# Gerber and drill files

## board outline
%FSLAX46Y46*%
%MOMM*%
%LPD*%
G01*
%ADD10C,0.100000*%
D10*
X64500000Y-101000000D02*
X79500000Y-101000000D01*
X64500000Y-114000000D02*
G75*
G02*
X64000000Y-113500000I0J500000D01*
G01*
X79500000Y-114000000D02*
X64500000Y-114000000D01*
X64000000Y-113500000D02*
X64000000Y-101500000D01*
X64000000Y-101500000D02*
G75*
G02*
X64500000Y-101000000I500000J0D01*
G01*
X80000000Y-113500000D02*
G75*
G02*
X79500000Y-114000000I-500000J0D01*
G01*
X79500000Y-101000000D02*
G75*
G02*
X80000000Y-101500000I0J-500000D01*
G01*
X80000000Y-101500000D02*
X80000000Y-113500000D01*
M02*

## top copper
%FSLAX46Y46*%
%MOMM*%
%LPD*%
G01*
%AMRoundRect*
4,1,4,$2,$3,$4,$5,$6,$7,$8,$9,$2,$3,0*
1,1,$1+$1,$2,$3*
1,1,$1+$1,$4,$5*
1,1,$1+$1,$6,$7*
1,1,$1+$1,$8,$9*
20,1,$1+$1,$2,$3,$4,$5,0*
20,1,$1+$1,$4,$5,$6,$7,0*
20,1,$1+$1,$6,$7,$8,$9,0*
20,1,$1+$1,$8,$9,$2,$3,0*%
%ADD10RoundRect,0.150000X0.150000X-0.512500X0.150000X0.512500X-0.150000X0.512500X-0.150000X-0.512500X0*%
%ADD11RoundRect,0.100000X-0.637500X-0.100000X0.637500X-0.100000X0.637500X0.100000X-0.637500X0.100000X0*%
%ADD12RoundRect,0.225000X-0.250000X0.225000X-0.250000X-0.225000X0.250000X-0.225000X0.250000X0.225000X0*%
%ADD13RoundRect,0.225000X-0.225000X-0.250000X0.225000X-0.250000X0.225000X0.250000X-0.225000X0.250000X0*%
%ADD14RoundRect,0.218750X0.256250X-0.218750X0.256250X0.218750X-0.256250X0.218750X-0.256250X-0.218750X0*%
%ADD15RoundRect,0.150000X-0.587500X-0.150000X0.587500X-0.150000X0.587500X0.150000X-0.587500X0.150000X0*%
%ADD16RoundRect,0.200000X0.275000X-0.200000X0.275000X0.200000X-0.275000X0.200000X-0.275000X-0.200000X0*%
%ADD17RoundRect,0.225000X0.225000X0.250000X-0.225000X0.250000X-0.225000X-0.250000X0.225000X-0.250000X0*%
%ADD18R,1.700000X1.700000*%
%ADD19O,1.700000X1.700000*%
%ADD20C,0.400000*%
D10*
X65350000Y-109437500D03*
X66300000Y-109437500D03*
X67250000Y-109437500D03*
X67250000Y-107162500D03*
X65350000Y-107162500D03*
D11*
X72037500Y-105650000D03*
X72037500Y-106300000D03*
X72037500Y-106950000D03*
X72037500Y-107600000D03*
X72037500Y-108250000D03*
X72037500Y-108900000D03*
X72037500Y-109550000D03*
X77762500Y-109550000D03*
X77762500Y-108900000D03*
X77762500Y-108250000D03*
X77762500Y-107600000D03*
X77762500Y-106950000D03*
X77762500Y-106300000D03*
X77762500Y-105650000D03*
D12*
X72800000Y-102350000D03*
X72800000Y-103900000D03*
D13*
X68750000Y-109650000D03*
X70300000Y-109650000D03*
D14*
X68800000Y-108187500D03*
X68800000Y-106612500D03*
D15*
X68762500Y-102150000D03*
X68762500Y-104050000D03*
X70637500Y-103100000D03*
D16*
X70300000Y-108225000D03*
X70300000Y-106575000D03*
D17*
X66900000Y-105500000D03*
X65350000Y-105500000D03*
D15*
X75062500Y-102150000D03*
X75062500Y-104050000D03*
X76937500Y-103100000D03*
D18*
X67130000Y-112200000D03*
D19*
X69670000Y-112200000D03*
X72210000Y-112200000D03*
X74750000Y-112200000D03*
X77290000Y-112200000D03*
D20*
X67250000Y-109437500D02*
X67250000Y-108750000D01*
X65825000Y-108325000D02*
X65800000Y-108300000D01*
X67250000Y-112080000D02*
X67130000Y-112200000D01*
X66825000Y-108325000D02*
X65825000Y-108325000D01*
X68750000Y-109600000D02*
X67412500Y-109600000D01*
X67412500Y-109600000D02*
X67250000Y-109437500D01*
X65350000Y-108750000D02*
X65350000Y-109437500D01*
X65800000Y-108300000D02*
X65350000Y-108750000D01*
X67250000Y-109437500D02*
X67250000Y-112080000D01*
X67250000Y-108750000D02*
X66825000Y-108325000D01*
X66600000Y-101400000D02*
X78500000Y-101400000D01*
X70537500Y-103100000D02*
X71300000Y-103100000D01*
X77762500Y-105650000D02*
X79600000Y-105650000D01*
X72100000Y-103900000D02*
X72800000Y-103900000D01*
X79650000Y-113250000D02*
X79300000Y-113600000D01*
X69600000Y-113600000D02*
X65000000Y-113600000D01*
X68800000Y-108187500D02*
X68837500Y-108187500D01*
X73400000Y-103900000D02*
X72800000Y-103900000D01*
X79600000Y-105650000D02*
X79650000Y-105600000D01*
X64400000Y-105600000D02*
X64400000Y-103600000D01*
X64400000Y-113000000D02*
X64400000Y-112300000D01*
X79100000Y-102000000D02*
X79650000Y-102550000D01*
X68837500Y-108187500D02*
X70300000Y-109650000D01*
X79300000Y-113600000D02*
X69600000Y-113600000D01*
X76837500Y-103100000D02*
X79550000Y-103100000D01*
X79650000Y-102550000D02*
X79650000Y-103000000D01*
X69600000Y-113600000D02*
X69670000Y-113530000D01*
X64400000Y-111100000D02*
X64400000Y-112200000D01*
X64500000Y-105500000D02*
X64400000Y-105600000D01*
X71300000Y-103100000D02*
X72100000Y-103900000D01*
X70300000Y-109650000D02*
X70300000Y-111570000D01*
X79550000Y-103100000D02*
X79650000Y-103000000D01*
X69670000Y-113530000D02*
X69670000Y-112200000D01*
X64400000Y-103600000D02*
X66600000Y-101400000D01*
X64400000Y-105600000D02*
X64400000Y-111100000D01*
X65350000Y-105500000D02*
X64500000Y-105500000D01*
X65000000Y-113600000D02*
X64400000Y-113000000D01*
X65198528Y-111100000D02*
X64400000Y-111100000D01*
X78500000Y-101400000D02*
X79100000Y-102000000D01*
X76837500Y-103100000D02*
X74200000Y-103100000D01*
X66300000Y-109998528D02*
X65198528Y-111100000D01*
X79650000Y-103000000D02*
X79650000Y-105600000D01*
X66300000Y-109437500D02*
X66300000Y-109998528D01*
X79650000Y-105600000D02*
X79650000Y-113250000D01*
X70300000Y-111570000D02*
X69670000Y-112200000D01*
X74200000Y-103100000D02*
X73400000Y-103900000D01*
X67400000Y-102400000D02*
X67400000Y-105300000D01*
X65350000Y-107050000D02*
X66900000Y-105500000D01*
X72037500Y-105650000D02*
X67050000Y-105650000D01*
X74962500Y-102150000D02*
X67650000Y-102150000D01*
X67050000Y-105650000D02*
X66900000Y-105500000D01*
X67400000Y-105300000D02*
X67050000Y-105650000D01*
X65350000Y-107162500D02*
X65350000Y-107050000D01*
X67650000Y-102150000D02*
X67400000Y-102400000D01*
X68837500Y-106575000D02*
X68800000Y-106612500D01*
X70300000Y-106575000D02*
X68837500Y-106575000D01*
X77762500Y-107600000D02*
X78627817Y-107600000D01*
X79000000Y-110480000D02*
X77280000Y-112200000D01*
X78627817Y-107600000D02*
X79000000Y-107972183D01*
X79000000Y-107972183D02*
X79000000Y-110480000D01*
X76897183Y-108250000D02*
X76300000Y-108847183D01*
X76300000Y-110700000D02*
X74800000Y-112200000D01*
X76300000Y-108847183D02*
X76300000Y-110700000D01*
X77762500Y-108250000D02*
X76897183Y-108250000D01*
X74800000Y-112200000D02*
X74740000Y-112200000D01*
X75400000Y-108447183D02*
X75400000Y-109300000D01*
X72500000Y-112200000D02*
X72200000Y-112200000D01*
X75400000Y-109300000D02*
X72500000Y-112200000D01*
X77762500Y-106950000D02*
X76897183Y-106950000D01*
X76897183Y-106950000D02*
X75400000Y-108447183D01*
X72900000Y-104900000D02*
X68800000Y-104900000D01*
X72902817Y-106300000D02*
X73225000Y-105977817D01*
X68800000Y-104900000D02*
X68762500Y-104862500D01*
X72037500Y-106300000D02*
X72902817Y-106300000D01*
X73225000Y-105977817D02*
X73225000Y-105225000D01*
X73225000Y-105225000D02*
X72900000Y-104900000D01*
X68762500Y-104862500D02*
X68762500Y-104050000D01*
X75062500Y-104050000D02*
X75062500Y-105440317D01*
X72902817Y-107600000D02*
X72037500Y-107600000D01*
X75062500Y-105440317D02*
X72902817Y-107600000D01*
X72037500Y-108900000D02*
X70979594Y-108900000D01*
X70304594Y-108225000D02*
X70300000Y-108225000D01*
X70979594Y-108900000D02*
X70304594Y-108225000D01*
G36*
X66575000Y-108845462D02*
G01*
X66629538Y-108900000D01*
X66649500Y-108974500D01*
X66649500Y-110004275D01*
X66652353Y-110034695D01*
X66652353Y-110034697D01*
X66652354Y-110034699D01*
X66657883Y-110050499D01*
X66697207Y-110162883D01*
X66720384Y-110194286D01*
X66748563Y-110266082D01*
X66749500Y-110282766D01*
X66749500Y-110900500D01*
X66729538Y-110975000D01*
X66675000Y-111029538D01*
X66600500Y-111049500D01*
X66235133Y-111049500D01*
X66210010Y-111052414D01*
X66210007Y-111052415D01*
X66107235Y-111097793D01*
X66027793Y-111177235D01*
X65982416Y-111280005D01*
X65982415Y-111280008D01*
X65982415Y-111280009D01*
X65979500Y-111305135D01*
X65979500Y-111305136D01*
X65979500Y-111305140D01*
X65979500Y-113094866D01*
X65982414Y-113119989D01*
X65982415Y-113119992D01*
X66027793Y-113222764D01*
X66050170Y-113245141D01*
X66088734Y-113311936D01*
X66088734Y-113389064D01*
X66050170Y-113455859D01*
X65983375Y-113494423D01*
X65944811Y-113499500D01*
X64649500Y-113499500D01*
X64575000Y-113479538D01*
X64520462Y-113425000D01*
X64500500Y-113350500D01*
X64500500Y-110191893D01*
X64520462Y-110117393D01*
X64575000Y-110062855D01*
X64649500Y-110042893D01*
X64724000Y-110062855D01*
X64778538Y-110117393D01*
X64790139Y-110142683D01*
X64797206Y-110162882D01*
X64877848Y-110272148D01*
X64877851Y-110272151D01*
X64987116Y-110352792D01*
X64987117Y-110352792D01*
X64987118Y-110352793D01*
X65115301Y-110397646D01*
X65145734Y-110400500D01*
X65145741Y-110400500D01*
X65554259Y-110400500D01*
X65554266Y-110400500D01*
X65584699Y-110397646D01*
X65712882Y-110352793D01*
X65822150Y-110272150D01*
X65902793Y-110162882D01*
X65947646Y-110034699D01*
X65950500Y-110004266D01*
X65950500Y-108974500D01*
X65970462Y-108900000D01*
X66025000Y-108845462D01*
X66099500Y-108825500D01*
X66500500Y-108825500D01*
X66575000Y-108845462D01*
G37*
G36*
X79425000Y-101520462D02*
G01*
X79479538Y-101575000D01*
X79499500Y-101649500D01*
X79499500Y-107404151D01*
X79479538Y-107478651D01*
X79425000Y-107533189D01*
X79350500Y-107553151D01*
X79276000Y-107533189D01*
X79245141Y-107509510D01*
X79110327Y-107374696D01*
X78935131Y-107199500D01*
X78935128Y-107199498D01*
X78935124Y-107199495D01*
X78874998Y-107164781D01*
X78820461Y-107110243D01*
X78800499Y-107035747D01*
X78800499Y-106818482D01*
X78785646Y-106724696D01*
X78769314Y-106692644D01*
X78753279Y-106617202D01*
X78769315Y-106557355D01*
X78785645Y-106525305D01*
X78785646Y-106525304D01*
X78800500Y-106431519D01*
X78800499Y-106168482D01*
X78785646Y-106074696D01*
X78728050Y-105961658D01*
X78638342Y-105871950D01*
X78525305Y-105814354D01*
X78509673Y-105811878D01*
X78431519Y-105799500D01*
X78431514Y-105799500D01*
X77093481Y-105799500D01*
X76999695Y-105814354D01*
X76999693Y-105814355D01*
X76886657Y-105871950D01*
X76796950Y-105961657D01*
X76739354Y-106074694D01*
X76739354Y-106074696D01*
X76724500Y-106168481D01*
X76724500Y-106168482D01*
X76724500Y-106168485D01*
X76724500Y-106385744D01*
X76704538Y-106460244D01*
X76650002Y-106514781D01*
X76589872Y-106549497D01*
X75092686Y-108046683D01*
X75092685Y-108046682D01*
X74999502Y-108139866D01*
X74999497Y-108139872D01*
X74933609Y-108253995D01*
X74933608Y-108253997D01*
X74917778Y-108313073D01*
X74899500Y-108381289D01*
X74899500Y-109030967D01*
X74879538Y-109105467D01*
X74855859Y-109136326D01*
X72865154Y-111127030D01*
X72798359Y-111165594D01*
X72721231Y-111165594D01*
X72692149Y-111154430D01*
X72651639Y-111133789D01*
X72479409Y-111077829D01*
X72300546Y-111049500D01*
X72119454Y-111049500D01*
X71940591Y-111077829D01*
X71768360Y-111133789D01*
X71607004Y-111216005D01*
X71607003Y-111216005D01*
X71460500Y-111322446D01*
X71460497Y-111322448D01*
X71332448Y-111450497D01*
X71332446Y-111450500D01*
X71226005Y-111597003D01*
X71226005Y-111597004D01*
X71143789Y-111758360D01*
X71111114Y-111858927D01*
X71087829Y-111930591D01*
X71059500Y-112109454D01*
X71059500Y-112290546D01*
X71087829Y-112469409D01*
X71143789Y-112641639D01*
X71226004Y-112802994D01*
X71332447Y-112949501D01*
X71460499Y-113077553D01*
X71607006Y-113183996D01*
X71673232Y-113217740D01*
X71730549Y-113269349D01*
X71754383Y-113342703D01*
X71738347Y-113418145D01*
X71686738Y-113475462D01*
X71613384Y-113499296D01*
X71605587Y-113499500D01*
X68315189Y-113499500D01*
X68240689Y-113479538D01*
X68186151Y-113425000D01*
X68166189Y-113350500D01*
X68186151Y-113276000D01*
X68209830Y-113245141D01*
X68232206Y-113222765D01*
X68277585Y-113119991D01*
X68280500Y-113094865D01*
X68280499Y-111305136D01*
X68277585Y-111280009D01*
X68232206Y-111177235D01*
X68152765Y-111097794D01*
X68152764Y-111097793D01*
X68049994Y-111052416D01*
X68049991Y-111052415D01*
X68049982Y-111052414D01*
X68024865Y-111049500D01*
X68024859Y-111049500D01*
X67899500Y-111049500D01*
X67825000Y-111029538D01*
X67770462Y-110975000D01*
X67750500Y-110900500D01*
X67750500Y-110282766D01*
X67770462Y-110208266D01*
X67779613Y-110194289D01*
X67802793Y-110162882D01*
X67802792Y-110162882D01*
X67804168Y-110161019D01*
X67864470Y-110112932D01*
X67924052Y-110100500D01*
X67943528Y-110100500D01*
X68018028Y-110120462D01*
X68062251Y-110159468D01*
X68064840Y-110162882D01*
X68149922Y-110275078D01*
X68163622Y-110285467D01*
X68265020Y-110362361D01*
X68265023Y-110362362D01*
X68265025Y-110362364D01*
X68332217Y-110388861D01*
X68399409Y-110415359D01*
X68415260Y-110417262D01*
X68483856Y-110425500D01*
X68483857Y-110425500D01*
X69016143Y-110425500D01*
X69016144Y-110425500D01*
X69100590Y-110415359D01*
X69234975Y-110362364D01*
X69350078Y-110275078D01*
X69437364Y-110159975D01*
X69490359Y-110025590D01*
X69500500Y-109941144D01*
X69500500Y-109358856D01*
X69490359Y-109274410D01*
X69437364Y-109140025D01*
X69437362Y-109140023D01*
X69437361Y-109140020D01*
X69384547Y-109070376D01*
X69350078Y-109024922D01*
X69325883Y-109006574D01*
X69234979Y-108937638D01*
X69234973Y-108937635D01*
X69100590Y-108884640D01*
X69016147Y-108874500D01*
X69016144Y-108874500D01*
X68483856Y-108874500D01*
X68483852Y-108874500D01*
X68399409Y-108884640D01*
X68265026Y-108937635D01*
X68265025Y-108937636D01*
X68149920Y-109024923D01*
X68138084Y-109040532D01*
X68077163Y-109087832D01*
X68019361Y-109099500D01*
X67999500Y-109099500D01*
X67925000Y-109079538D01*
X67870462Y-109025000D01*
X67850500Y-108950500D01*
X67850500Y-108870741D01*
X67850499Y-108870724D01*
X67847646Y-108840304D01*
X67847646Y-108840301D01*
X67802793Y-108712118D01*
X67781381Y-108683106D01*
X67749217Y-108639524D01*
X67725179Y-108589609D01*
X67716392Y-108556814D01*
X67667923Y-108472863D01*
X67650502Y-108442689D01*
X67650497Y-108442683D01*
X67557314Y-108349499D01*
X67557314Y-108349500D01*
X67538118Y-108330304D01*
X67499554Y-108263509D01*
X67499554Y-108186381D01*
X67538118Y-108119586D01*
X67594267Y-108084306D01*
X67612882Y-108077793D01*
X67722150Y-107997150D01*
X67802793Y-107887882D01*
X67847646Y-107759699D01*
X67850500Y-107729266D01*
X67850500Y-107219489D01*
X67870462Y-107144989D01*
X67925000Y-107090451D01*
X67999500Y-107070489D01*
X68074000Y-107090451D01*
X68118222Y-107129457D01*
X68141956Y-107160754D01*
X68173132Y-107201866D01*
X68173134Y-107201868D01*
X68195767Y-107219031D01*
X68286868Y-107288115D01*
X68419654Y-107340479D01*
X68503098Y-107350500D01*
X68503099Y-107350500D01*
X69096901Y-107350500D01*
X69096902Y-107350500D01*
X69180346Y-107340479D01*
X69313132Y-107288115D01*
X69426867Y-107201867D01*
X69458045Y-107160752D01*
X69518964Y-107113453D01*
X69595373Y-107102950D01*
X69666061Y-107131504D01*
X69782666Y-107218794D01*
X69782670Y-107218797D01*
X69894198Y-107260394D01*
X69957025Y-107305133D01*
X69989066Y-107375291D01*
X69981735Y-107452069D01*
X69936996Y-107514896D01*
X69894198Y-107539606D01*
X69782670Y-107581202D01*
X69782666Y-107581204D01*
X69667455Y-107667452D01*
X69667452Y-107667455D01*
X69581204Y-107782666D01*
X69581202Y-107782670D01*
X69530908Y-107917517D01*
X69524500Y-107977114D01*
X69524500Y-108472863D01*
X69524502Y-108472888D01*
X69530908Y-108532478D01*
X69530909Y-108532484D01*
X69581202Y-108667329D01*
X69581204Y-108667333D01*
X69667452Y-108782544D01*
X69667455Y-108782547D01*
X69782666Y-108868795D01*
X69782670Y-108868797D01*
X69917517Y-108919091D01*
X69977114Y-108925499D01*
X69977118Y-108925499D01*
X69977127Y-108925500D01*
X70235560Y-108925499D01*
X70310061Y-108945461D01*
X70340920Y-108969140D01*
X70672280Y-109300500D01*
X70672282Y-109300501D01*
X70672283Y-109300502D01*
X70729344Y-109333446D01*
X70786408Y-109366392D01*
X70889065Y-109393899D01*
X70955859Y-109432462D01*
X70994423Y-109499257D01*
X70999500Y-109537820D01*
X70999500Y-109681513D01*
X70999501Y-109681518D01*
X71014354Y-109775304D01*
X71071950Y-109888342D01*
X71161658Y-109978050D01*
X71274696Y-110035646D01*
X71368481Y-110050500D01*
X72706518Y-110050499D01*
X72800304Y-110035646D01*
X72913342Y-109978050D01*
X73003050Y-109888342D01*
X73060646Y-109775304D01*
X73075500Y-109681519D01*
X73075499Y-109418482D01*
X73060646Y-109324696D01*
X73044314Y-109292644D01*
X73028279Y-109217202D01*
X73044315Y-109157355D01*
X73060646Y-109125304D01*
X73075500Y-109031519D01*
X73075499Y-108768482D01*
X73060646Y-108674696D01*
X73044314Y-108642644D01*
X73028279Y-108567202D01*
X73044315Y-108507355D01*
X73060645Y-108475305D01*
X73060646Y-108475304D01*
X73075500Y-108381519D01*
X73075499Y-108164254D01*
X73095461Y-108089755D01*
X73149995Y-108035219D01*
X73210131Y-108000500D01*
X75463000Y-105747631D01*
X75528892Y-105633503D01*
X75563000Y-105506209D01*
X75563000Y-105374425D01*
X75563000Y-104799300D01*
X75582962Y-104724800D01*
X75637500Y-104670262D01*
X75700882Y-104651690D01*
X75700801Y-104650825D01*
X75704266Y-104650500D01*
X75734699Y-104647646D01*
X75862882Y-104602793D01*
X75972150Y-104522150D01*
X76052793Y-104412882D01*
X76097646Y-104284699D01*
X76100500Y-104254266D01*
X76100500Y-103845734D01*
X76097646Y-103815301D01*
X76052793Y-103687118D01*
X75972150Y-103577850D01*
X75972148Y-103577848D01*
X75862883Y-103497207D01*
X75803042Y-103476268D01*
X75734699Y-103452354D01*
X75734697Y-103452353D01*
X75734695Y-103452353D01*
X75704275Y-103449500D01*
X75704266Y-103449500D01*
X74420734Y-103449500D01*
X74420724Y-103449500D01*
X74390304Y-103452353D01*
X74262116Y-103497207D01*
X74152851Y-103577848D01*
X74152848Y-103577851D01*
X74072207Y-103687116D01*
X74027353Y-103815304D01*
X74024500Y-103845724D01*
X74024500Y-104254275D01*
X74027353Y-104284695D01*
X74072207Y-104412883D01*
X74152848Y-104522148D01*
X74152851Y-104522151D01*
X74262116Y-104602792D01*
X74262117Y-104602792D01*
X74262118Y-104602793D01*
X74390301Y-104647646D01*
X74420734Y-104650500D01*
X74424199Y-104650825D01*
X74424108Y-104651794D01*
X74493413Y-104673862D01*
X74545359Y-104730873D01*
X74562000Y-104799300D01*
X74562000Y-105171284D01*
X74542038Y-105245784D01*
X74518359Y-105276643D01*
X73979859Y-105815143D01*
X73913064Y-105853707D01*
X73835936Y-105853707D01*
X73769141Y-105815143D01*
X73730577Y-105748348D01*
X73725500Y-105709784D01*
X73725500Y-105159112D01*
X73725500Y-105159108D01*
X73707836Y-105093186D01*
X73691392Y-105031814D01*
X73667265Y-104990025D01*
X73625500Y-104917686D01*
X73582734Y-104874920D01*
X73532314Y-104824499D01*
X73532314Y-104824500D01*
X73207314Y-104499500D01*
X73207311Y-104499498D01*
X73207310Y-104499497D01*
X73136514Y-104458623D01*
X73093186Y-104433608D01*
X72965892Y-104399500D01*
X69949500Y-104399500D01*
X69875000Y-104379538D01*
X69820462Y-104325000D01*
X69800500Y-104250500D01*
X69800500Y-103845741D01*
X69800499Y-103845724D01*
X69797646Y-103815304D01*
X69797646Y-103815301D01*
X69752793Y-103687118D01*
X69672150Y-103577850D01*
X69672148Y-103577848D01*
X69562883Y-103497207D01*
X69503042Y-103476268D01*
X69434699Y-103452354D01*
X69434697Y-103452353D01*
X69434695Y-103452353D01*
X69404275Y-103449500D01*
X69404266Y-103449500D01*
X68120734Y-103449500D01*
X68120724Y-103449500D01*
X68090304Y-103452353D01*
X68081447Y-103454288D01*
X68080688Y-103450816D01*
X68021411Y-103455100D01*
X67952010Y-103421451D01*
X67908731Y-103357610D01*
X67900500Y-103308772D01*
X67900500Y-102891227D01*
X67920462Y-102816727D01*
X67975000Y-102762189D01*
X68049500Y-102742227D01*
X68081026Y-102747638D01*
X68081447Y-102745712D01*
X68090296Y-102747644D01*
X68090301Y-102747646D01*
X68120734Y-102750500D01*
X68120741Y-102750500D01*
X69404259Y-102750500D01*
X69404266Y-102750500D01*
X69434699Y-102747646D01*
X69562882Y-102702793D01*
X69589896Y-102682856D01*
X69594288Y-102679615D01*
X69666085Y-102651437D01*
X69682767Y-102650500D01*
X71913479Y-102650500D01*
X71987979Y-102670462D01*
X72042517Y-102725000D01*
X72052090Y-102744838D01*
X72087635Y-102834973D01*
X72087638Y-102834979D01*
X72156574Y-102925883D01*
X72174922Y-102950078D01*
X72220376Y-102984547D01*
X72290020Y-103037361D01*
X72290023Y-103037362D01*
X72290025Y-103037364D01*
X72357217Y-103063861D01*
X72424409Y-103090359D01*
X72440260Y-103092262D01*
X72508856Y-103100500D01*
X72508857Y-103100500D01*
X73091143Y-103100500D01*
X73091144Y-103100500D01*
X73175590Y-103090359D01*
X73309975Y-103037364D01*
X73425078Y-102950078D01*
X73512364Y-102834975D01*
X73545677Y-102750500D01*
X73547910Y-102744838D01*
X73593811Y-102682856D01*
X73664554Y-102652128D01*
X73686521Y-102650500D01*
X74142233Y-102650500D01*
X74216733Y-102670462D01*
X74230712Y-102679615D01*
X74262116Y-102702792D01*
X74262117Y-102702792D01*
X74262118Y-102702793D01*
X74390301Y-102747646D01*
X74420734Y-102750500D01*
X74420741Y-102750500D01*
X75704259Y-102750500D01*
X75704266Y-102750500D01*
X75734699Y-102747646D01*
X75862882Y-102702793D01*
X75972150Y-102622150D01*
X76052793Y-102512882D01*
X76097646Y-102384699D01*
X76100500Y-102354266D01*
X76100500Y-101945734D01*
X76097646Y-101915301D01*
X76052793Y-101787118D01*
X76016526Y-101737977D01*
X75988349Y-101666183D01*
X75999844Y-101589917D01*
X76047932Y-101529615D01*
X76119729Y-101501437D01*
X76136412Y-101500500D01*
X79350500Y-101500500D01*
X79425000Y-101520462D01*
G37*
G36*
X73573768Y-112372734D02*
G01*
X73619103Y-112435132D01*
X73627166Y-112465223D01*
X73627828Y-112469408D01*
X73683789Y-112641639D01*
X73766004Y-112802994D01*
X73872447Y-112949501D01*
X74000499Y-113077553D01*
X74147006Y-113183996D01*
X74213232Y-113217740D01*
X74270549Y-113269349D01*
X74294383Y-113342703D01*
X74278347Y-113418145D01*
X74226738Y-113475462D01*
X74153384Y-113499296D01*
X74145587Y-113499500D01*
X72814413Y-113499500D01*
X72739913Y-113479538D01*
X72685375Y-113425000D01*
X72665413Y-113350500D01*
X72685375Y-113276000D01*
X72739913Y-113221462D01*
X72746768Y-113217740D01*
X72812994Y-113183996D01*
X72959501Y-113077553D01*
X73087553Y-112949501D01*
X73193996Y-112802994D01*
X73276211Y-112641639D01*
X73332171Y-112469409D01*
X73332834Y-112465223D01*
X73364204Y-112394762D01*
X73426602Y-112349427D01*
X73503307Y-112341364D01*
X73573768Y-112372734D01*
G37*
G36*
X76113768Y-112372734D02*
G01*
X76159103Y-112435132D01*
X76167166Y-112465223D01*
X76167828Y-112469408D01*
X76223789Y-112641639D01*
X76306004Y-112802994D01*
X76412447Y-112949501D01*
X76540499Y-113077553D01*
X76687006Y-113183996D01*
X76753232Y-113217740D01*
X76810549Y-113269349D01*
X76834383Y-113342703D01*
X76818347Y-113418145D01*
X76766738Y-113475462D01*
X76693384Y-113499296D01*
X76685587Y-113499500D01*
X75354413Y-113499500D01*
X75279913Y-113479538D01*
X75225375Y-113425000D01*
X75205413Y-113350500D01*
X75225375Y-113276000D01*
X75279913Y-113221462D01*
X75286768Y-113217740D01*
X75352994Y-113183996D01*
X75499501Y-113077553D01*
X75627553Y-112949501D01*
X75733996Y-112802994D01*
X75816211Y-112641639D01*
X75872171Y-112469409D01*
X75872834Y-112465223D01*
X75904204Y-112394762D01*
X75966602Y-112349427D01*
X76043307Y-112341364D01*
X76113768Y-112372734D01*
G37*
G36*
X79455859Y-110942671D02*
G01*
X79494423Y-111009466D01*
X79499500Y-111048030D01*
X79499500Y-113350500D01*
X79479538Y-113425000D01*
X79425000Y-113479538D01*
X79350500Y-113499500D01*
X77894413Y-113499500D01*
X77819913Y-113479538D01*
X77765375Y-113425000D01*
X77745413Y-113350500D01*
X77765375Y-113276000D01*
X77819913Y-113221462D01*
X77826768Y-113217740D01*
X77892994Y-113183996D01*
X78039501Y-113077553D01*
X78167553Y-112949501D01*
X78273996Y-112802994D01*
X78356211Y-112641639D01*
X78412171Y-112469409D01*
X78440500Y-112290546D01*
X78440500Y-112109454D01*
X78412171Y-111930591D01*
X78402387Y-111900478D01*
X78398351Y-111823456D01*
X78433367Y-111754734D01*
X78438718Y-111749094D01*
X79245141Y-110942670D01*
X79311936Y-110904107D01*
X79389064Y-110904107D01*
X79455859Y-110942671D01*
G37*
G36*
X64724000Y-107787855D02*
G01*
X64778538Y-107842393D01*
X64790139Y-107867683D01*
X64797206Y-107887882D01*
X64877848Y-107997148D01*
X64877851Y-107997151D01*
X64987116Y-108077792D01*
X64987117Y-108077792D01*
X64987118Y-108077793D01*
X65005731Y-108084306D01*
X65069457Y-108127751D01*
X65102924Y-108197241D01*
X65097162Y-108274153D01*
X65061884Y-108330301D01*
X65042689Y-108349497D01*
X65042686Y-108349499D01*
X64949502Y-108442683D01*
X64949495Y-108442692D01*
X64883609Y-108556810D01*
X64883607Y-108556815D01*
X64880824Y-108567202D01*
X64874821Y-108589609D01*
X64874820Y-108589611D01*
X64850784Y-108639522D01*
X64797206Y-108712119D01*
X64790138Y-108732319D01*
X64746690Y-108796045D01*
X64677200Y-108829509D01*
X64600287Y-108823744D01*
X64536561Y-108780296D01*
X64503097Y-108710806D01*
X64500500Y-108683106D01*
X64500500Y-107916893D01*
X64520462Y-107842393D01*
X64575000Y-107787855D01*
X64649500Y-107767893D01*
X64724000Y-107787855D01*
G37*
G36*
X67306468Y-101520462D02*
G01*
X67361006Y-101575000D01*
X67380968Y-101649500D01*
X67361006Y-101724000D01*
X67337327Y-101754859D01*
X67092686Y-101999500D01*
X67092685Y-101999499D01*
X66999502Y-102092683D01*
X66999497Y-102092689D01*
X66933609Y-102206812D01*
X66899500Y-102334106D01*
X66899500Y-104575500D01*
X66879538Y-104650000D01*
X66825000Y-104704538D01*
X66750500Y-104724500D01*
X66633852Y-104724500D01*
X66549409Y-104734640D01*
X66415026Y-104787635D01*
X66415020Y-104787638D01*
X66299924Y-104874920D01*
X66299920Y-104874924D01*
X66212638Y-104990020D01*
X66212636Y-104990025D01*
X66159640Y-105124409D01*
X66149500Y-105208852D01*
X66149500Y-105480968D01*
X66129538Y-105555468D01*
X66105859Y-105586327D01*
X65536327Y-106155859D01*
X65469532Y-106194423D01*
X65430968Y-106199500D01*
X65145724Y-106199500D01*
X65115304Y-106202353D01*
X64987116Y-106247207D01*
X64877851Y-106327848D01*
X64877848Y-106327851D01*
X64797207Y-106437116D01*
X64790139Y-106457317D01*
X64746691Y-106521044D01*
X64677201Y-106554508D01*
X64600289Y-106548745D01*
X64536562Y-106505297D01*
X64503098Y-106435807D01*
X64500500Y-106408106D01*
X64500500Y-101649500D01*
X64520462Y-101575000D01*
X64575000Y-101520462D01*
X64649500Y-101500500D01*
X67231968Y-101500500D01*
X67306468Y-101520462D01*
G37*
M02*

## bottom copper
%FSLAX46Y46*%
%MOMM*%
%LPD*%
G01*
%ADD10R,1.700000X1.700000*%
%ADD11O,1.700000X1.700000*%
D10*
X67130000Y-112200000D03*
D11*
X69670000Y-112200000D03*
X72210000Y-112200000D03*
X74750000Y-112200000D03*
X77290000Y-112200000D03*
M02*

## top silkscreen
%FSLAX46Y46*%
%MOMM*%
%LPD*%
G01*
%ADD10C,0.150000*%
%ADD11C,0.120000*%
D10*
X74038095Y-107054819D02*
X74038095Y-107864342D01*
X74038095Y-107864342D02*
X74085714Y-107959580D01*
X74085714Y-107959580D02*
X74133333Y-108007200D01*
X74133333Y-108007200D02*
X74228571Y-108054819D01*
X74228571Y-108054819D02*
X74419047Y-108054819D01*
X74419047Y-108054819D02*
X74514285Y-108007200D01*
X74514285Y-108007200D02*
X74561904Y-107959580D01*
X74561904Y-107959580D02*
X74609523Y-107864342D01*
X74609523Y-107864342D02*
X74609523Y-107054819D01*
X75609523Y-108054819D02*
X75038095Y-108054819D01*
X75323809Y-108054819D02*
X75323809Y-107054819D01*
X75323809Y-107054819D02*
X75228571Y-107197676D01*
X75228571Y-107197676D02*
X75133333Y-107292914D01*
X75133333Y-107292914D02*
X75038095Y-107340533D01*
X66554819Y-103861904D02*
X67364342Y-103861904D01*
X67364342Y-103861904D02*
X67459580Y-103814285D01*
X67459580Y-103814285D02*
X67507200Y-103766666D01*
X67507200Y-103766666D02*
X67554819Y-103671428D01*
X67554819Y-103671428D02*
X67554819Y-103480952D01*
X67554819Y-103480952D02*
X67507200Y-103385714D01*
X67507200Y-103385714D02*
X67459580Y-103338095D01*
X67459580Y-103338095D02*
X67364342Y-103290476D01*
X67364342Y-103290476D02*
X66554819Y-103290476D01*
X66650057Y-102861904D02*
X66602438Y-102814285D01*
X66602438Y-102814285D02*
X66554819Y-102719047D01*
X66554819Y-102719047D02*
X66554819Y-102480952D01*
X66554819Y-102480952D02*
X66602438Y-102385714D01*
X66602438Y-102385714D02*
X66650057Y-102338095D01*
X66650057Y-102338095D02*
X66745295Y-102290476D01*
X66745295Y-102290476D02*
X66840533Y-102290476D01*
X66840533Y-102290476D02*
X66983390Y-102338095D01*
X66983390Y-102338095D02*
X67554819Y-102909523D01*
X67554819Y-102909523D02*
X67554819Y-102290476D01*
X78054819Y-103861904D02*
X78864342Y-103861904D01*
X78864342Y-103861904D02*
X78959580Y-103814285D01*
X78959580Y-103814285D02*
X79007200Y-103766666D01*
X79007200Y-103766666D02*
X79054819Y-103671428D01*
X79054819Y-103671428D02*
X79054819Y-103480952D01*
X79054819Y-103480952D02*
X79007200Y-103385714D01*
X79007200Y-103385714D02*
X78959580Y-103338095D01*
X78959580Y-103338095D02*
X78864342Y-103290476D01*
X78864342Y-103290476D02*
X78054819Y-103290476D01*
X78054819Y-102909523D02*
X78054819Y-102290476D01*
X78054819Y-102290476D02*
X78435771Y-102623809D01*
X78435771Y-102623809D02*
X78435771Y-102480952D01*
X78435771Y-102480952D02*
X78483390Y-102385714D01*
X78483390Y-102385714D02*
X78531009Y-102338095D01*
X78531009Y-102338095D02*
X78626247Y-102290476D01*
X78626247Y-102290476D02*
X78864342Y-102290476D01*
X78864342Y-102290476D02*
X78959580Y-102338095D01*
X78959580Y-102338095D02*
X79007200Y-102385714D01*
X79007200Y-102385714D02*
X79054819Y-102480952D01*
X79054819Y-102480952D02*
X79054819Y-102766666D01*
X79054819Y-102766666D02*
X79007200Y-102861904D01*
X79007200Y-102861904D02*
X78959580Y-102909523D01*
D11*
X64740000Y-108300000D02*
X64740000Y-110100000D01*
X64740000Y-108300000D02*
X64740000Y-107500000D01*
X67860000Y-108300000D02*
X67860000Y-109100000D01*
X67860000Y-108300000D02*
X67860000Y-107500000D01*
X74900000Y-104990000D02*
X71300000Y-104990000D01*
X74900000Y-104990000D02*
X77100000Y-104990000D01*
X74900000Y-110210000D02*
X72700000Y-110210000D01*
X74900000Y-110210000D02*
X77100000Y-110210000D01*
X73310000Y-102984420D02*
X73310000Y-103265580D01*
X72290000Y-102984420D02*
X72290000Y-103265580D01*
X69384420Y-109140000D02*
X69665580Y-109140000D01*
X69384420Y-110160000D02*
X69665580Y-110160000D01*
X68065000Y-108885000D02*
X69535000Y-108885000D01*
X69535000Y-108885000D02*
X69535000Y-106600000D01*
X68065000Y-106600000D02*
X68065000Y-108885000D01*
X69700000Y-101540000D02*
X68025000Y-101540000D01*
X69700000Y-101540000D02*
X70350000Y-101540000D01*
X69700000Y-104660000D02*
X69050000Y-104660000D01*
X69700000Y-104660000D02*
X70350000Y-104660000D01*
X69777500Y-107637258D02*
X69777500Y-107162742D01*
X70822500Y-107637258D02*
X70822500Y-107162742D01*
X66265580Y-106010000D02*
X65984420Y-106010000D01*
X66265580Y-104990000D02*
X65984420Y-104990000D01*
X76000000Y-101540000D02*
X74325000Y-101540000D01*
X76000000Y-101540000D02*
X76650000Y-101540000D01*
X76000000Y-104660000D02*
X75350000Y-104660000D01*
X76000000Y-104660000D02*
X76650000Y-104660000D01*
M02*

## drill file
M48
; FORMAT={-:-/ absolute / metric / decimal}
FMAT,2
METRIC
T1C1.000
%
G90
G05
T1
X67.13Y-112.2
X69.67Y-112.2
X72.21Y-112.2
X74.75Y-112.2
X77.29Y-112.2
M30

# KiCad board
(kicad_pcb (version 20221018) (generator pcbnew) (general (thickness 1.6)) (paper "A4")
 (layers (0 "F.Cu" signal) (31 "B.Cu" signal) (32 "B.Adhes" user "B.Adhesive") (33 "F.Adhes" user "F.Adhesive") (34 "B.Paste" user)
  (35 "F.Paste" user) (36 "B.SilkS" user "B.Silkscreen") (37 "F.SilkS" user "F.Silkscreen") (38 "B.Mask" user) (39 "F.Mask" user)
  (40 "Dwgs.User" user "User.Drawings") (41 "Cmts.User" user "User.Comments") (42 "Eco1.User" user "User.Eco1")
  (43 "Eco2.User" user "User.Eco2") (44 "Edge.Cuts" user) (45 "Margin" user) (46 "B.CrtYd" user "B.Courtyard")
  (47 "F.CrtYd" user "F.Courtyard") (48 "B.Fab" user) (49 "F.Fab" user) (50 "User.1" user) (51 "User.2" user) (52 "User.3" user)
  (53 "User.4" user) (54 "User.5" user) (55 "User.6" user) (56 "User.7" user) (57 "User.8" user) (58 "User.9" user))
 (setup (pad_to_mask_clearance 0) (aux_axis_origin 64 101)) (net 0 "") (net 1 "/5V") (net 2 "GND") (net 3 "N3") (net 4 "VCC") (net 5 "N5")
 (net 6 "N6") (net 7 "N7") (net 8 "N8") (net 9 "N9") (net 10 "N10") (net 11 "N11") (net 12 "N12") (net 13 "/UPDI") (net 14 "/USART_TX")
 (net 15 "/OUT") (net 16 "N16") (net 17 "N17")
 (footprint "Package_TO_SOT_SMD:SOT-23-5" (layer "F.Cu") (at 66.3 108.3 90)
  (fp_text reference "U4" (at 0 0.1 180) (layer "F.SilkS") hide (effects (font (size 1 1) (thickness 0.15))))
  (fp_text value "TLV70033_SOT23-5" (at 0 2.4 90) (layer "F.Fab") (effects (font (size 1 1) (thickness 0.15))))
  (fp_line (start 0 -1.56) (end -1.8 -1.56) (stroke (width 0.12) (type solid)) (layer "F.SilkS"))
  (fp_line (start 0 -1.56) (end 0.8 -1.56) (stroke (width 0.12) (type solid)) (layer "F.SilkS"))
  (fp_line (start 0 1.56) (end -0.8 1.56) (stroke (width 0.12) (type solid)) (layer "F.SilkS"))
  (fp_line (start 0 1.56) (end 0.8 1.56) (stroke (width 0.12) (type solid)) (layer "F.SilkS"))
  (pad "1" smd roundrect (at -1.1375 -0.95 90) (size 1.325 0.6) (layers "F.Cu" "F.Paste" "F.Mask") (roundrect_rratio 0.25) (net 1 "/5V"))
  (pad "2" smd roundrect (at -1.1375 0 90) (size 1.325 0.6) (layers "F.Cu" "F.Paste" "F.Mask") (roundrect_rratio 0.25) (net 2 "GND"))
  (pad "3" smd roundrect (at -1.1375 0.95 90) (size 1.325 0.6) (layers "F.Cu" "F.Paste" "F.Mask") (roundrect_rratio 0.25) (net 1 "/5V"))
  (pad "4" smd roundrect (at 1.1375 0.95 90) (size 1.325 0.6) (layers "F.Cu" "F.Paste" "F.Mask") (roundrect_rratio 0.25) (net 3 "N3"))
  (pad "5" smd roundrect (at 1.1375 -0.95 90) (size 1.325 0.6) (layers "F.Cu" "F.Paste" "F.Mask") (roundrect_rratio 0.25) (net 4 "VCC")))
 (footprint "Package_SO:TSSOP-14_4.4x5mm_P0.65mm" (layer "F.Cu") (at 74.9 107.6)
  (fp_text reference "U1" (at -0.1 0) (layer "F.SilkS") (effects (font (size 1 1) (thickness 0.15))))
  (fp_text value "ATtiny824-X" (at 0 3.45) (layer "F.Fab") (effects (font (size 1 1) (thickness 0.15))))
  (fp_line (start 0 -2.61) (end -3.6 -2.61) (stroke (width 0.12) (type solid)) (layer "F.SilkS"))
  (fp_line (start 0 -2.61) (end 2.2 -2.61) (stroke (width 0.12) (type solid)) (layer "F.SilkS"))
  (fp_line (start 0 2.61) (end -2.2 2.61) (stroke (width 0.12) (type solid)) (layer "F.SilkS"))
  (fp_line (start 0 2.61) (end 2.2 2.61) (stroke (width 0.12) (type solid)) (layer "F.SilkS"))
  (pad "1" smd roundrect (at -2.8625 -1.95) (size 1.475 0.4) (layers "F.Cu" "F.Paste" "F.Mask") (roundrect_rratio 0.25) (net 4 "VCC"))
  (pad "2" smd roundrect (at -2.8625 -1.3) (size 1.475 0.4) (layers "F.Cu" "F.Paste" "F.Mask") (roundrect_rratio 0.25) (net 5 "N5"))
  (pad "3" smd roundrect (at -2.8625 -0.65) (size 1.475 0.4) (layers "F.Cu" "F.Paste" "F.Mask") (roundrect_rratio 0.25) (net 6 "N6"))
  (pad "4" smd roundrect (at -2.8625 0) (size 1.475 0.4) (layers "F.Cu" "F.Paste" "F.Mask") (roundrect_rratio 0.25) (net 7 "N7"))
  (pad "5" smd roundrect (at -2.8625 0.65) (size 1.475 0.4) (layers "F.Cu" "F.Paste" "F.Mask") (roundrect_rratio 0.25) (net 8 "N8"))
  (pad "6" smd roundrect (at -2.8625 1.3) (size 1.475 0.4) (layers "F.Cu" "F.Paste" "F.Mask") (roundrect_rratio 0.25) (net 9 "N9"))
  (pad "7" smd roundrect (at -2.8625 1.95) (size 1.475 0.4) (layers "F.Cu" "F.Paste" "F.Mask") (roundrect_rratio 0.25) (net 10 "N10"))
  (pad "8" smd roundrect (at 2.8625 1.95) (size 1.475 0.4) (layers "F.Cu" "F.Paste" "F.Mask") (roundrect_rratio 0.25) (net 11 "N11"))
  (pad "9" smd roundrect (at 2.8625 1.3) (size 1.475 0.4) (layers "F.Cu" "F.Paste" "F.Mask") (roundrect_rratio 0.25) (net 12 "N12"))
  (pad "10" smd roundrect (at 2.8625 0.65) (size 1.475 0.4) (layers "F.Cu" "F.Paste" "F.Mask") (roundrect_rratio 0.25) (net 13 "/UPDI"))
  (pad "11" smd roundrect (at 2.8625 0) (size 1.475 0.4) (layers "F.Cu" "F.Paste" "F.Mask") (roundrect_rratio 0.25) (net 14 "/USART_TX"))
  (pad "12" smd roundrect (at 2.8625 -0.65) (size 1.475 0.4) (layers "F.Cu" "F.Paste" "F.Mask") (roundrect_rratio 0.25) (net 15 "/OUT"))
  (pad "13" smd roundrect (at 2.8625 -1.3) (size 1.475 0.4) (layers "F.Cu" "F.Paste" "F.Mask") (roundrect_rratio 0.25) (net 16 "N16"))
  (pad "14" smd roundrect (at 2.8625 -1.95) (size 1.475 0.4) (layers "F.Cu" "F.Paste" "F.Mask") (roundrect_rratio 0.25) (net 2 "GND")))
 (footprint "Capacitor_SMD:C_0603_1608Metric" (layer "F.Cu") (at 72.8 103.125 -90)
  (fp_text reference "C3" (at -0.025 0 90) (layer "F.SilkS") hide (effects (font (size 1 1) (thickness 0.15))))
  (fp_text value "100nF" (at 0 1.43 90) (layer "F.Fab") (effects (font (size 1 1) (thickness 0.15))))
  (fp_line (start -0.14058 -0.51) (end 0.14058 -0.51) (stroke (width 0.12) (type solid)) (layer "F.SilkS"))
  (fp_line (start -0.14058 0.51) (end 0.14058 0.51) (stroke (width 0.12) (type solid)) (layer "F.SilkS"))
  (pad "1" smd roundrect (at -0.775 0 270) (size 0.9 0.95) (layers "F.Cu" "F.Paste" "F.Mask") (roundrect_rratio 0.25) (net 4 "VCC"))
  (pad "2" smd roundrect (at 0.775 0 270) (size 0.9 0.95) (layers "F.Cu" "F.Paste" "F.Mask") (roundrect_rratio 0.25) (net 2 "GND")))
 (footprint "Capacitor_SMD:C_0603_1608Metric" (layer "F.Cu") (at 69.525 109.65)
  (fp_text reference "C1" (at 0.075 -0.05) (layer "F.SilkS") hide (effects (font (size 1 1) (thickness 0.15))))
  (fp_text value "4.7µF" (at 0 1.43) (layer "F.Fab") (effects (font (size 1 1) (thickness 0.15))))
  (fp_line (start -0.14058 -0.51) (end 0.14058 -0.51) (stroke (width 0.12) (type solid)) (layer "F.SilkS"))
  (fp_line (start -0.14058 0.51) (end 0.14058 0.51) (stroke (width 0.12) (type solid)) (layer "F.SilkS"))
  (pad "1" smd roundrect (at -0.775 0) (size 0.9 0.95) (layers "F.Cu" "F.Paste" "F.Mask") (roundrect_rratio 0.25) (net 1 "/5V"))
  (pad "2" smd roundrect (at 0.775 0) (size 0.9 0.95) (layers "F.Cu" "F.Paste" "F.Mask") (roundrect_rratio 0.25) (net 2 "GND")))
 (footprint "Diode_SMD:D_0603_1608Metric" (layer "F.Cu") (at 68.8 107.4 90)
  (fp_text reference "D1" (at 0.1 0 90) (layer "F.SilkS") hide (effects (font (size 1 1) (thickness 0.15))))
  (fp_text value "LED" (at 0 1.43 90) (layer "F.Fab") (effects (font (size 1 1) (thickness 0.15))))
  (fp_line (start -1.485 -0.735) (end -1.485 0.735) (stroke (width 0.12) (type solid)) (layer "F.SilkS"))
  (fp_line (start -1.485 0.735) (end 0.8 0.735) (stroke (width 0.12) (type solid)) (layer "F.SilkS"))
  (fp_line (start 0.8 -0.735) (end -1.485 -0.735) (stroke (width 0.12) (type solid)) (layer "F.SilkS"))
  (pad "1" smd roundrect (at -0.7875 0 90) (size 0.875 0.95) (layers "F.Cu" "F.Paste" "F.Mask") (roundrect_rratio 0.25) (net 2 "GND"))
  (pad "2" smd roundrect (at 0.7875 0 90) (size 0.875 0.95) (layers "F.Cu" "F.Paste" "F.Mask") (roundrect_rratio 0.25) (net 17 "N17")))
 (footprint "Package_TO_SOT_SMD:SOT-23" (layer "F.Cu") (at 69.7 103.1)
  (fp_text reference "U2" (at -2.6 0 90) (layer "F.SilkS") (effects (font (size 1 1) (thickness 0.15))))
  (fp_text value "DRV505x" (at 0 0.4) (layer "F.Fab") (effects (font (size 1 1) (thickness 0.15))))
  (fp_line (start 0 -1.56) (end -1.675 -1.56) (stroke (width 0.12) (type solid)) (layer "F.SilkS"))
  (fp_line (start 0 -1.56) (end 0.65 -1.56) (stroke (width 0.12) (type solid)) (layer "F.SilkS"))
  (fp_line (start 0 1.56) (end -0.65 1.56) (stroke (width 0.12) (type solid)) (layer "F.SilkS"))
  (fp_line (start 0 1.56) (end 0.65 1.56) (stroke (width 0.12) (type solid)) (layer "F.SilkS"))
  (pad "1" smd roundrect (at -0.9375 -0.95) (size 1.475 0.6) (layers "F.Cu" "F.Paste" "F.Mask") (roundrect_rratio 0.25) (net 4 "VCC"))
  (pad "2" smd roundrect (at -0.9375 0.95) (size 1.475 0.6) (layers "F.Cu" "F.Paste" "F.Mask") (roundrect_rratio 0.25) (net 5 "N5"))
  (pad "3" smd roundrect (at 0.9375 0) (size 1.475 0.6) (layers "F.Cu" "F.Paste" "F.Mask") (roundrect_rratio 0.25) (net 2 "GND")))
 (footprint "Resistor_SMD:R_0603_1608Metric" (layer "F.Cu") (at 70.3 107.4 90)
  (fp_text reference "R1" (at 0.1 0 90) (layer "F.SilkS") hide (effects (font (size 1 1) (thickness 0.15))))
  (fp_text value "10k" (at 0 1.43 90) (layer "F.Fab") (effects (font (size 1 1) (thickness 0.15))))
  (fp_line (start -0.237258 -0.5225) (end 0.237258 -0.5225) (stroke (width 0.12) (type solid)) (layer "F.SilkS"))
  (fp_line (start -0.237258 0.5225) (end 0.237258 0.5225) (stroke (width 0.12) (type solid)) (layer "F.SilkS"))
  (pad "1" smd roundrect (at -0.825 0 90) (size 0.8 0.95) (layers "F.Cu" "F.Paste" "F.Mask") (roundrect_rratio 0.25) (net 9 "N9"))
  (pad "2" smd roundrect (at 0.825 0 90) (size 0.8 0.95) (layers "F.Cu" "F.Paste" "F.Mask") (roundrect_rratio 0.25) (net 17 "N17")))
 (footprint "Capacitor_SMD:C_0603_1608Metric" (layer "F.Cu") (at 66.125 105.5 180)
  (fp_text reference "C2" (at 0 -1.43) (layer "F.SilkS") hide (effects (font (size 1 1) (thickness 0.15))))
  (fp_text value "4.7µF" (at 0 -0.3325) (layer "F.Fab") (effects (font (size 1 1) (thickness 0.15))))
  (fp_line (start -0.14058 -0.51) (end 0.14058 -0.51) (stroke (width 0.12) (type solid)) (layer "F.SilkS"))
  (fp_line (start -0.14058 0.51) (end 0.14058 0.51) (stroke (width 0.12) (type solid)) (layer "F.SilkS"))
  (pad "1" smd roundrect (at -0.775 0 180) (size 0.9 0.95) (layers "F.Cu" "F.Paste" "F.Mask") (roundrect_rratio 0.25) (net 4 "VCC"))
  (pad "2" smd roundrect (at 0.775 0 180) (size 0.9 0.95) (layers "F.Cu" "F.Paste" "F.Mask") (roundrect_rratio 0.25) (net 2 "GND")))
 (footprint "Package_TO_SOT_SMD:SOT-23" (layer "F.Cu") (at 76 103.1)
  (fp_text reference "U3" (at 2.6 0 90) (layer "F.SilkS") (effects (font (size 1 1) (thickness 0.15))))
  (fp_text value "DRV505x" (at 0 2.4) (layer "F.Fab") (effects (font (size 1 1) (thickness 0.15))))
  (fp_line (start 0 -1.56) (end -1.675 -1.56) (stroke (width 0.12) (type solid)) (layer "F.SilkS"))
  (fp_line (start 0 -1.56) (end 0.65 -1.56) (stroke (width 0.12) (type solid)) (layer "F.SilkS"))
  (fp_line (start 0 1.56) (end -0.65 1.56) (stroke (width 0.12) (type solid)) (layer "F.SilkS"))
  (fp_line (start 0 1.56) (end 0.65 1.56) (stroke (width 0.12) (type solid)) (layer "F.SilkS"))
  (pad "1" smd roundrect (at -0.9375 -0.95) (size 1.475 0.6) (layers "F.Cu" "F.Paste" "F.Mask") (roundrect_rratio 0.25) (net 4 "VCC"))
  (pad "2" smd roundrect (at -0.9375 0.95) (size 1.475 0.6) (layers "F.Cu" "F.Paste" "F.Mask") (roundrect_rratio 0.25) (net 7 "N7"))
  (pad "3" smd roundrect (at 0.9375 0) (size 1.475 0.6) (layers "F.Cu" "F.Paste" "F.Mask") (roundrect_rratio 0.25) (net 2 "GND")))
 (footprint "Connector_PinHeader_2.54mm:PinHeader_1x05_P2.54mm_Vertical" (layer "B.Cu") (at 67.13 112.2 -90)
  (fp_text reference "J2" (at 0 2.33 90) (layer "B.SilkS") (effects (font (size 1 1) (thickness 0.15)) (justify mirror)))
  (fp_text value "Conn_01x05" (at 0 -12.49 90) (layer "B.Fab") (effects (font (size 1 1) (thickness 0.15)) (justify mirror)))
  (pad "1" thru_hole rect (at 0 0 270) (size 1.7 1.7) (drill 1) (layers "*.Cu" "*.Mask") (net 1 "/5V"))
  (pad "2" thru_hole oval (at 0 -2.54 270) (size 1.7 1.7) (drill 1) (layers "*.Cu" "*.Mask") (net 2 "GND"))
  (pad "3" thru_hole oval (at 0 -5.08 270) (size 1.7 1.7) (drill 1) (layers "*.Cu" "*.Mask") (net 15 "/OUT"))
  (pad "4" thru_hole oval (at 0 -7.62 270) (size 1.7 1.7) (drill 1) (layers "*.Cu" "*.Mask") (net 13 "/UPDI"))
  (pad "5" thru_hole oval (at 0 -10.16 270) (size 1.7 1.7) (drill 1) (layers "*.Cu" "*.Mask") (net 14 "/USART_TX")))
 (gr_line (start 64.5 101) (end 79.5 101) (stroke (width 0.1) (type default)) (layer "Edge.Cuts"))
 (gr_arc (start 64.5 114) (mid 64.146447 113.853553) (end 64 113.5) (stroke (width 0.1) (type default)) (layer "Edge.Cuts"))
 (gr_line (start 79.5 114) (end 64.5 114) (stroke (width 0.1) (type default)) (layer "Edge.Cuts"))
 (gr_line (start 64 113.5) (end 64 101.5) (stroke (width 0.1) (type default)) (layer "Edge.Cuts"))
 (gr_arc (start 64 101.5) (mid 64.146447 101.146447) (end 64.5 101) (stroke (width 0.1) (type default)) (layer "Edge.Cuts"))
 (gr_arc (start 80 113.5) (mid 79.853553 113.853553) (end 79.5 114) (stroke (width 0.1) (type default)) (layer "Edge.Cuts"))
 (gr_arc (start 79.5 101) (mid 79.853553 101.146447) (end 80 101.5) (stroke (width 0.1) (type default)) (layer "Edge.Cuts"))
 (gr_line (start 80 101.5) (end 80 113.5) (stroke (width 0.1) (type default)) (layer "Edge.Cuts"))
 (segment (start 67.25 109.4375) (end 67.25 108.75) (width 0.4) (layer "F.Cu") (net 1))
 (segment (start 65.825 108.325) (end 65.8 108.3) (width 0.4) (layer "F.Cu") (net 1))
 (segment (start 67.25 112.08) (end 67.13 112.2) (width 0.4) (layer "F.Cu") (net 1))
 (segment (start 66.825 108.325) (end 65.825 108.325) (width 0.4) (layer "F.Cu") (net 1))
 (segment (start 68.75 109.6) (end 67.4125 109.6) (width 0.4) (layer "F.Cu") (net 1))
 (segment (start 67.4125 109.6) (end 67.25 109.4375) (width 0.4) (layer "F.Cu") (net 1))
 (segment (start 65.35 108.75) (end 65.35 109.4375) (width 0.4) (layer "F.Cu") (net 1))
 (segment (start 65.8 108.3) (end 65.35 108.75) (width 0.4) (layer "F.Cu") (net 1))
 (segment (start 67.25 109.4375) (end 67.25 112.08) (width 0.4) (layer "F.Cu") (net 1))
 (segment (start 67.25 108.75) (end 66.825 108.325) (width 0.4) (layer "F.Cu") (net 1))
 (segment (start 66.6 101.4) (end 78.5 101.4) (width 0.4) (layer "F.Cu") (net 2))
 (segment (start 70.5375 103.1) (end 71.3 103.1) (width 0.4) (layer "F.Cu") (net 2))
 (segment (start 77.7625 105.65) (end 79.6 105.65) (width 0.4) (layer "F.Cu") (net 2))
 (segment (start 72.1 103.9) (end 72.8 103.9) (width 0.4) (layer "F.Cu") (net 2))
 (segment (start 79.65 113.25) (end 79.3 113.6) (width 0.4) (layer "F.Cu") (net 2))
 (segment (start 69.6 113.6) (end 65 113.6) (width 0.4) (layer "F.Cu") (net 2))
 (segment (start 68.8 108.1875) (end 68.8375 108.1875) (width 0.4) (layer "F.Cu") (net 2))
 (segment (start 73.4 103.9) (end 72.8 103.9) (width 0.4) (layer "F.Cu") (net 2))
 (segment (start 79.6 105.65) (end 79.65 105.6) (width 0.4) (layer "F.Cu") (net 2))
 (segment (start 64.4 105.6) (end 64.4 103.6) (width 0.4) (layer "F.Cu") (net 2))
 (segment (start 64.4 113) (end 64.4 112.3) (width 0.4) (layer "F.Cu") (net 2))
 (segment (start 79.1 102) (end 79.65 102.55) (width 0.4) (layer "F.Cu") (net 2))
 (segment (start 68.8375 108.1875) (end 70.3 109.65) (width 0.4) (layer "F.Cu") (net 2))
 (segment (start 79.3 113.6) (end 69.6 113.6) (width 0.4) (layer "F.Cu") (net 2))
 (segment (start 76.8375 103.1) (end 79.55 103.1) (width 0.4) (layer "F.Cu") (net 2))
 (segment (start 79.65 102.55) (end 79.65 103) (width 0.4) (layer "F.Cu") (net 2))
 (segment (start 69.6 113.6) (end 69.67 113.53) (width 0.4) (layer "F.Cu") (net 2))
 (segment (start 64.4 111.1) (end 64.4 112.2) (width 0.4) (layer "F.Cu") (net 2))
 (segment (start 64.5 105.5) (end 64.4 105.6) (width 0.4) (layer "F.Cu") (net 2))
 (segment (start 71.3 103.1) (end 72.1 103.9) (width 0.4) (layer "F.Cu") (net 2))
 (segment (start 70.3 109.65) (end 70.3 111.57) (width 0.4) (layer "F.Cu") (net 2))
 (segment (start 79.55 103.1) (end 79.65 103) (width 0.4) (layer "F.Cu") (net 2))
 (segment (start 69.67 113.53) (end 69.67 112.2) (width 0.4) (layer "F.Cu") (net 2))
 (segment (start 64.4 103.6) (end 66.6 101.4) (width 0.4) (layer "F.Cu") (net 2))
 (segment (start 64.4 105.6) (end 64.4 111.1) (width 0.4) (layer "F.Cu") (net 2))
 (segment (start 65.35 105.5) (end 64.5 105.5) (width 0.4) (layer "F.Cu") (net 2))
 (segment (start 65 113.6) (end 64.4 113) (width 0.4) (layer "F.Cu") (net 2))
 (segment (start 65.198528 111.1) (end 64.4 111.1) (width 0.4) (layer "F.Cu") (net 2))
 (segment (start 78.5 101.4) (end 79.1 102) (width 0.4) (layer "F.Cu") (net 2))
 (segment (start 76.8375 103.1) (end 74.2 103.1) (width 0.4) (layer "F.Cu") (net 2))
 (segment (start 66.3 109.998528) (end 65.198528 111.1) (width 0.4) (layer "F.Cu") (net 2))
 (segment (start 79.65 103) (end 79.65 105.6) (width 0.4) (layer "F.Cu") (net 2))
 (segment (start 66.3 109.4375) (end 66.3 109.998528) (width 0.4) (layer "F.Cu") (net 2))
 (segment (start 79.65 105.6) (end 79.65 113.25) (width 0.4) (layer "F.Cu") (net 2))
 (segment (start 70.3 111.57) (end 69.67 112.2) (width 0.4) (layer "F.Cu") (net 2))
 (segment (start 74.2 103.1) (end 73.4 103.9) (width 0.4) (layer "F.Cu") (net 2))
 (segment (start 67.4 102.4) (end 67.4 105.3) (width 0.4) (layer "F.Cu") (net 4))
 (segment (start 65.35 107.05) (end 66.9 105.5) (width 0.4) (layer "F.Cu") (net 4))
 (segment (start 72.0375 105.65) (end 67.05 105.65) (width 0.4) (layer "F.Cu") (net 4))
 (segment (start 74.9625 102.15) (end 67.65 102.15) (width 0.4) (layer "F.Cu") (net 4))
 (segment (start 67.05 105.65) (end 66.9 105.5) (width 0.4) (layer "F.Cu") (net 4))
 (segment (start 67.4 105.3) (end 67.05 105.65) (width 0.4) (layer "F.Cu") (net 4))
 (segment (start 65.35 107.1625) (end 65.35 107.05) (width 0.4) (layer "F.Cu") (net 4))
 (segment (start 67.65 102.15) (end 67.4 102.4) (width 0.4) (layer "F.Cu") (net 4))
 (segment (start 68.8375 106.575) (end 68.8 106.6125) (width 0.4) (layer "F.Cu") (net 17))
 (segment (start 70.3 106.575) (end 68.8375 106.575) (width 0.4) (layer "F.Cu") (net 17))
 (segment (start 77.7625 107.6) (end 78.627817 107.6) (width 0.4) (layer "F.Cu") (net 14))
 (segment (start 79 110.48) (end 77.28 112.2) (width 0.4) (layer "F.Cu") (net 14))
 (segment (start 78.627817 107.6) (end 79 107.972183) (width 0.4) (layer "F.Cu") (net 14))
 (segment (start 79 107.972183) (end 79 110.48) (width 0.4) (layer "F.Cu") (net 14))
 (segment (start 76.897183 108.25) (end 76.3 108.847183) (width 0.4) (layer "F.Cu") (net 13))
 (segment (start 76.3 110.7) (end 74.8 112.2) (width 0.4) (layer "F.Cu") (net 13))
 (segment (start 76.3 108.847183) (end 76.3 110.7) (width 0.4) (layer "F.Cu") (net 13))
 (segment (start 77.7625 108.25) (end 76.897183 108.25) (width 0.4) (layer "F.Cu") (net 13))
 (segment (start 74.8 112.2) (end 74.74 112.2) (width 0.4) (layer "F.Cu") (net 13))
 (segment (start 75.4 108.447183) (end 75.4 109.3) (width 0.4) (layer "F.Cu") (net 15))
 (segment (start 72.5 112.2) (end 72.2 112.2) (width 0.4) (layer "F.Cu") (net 15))
 (segment (start 75.4 109.3) (end 72.5 112.2) (width 0.4) (layer "F.Cu") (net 15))
 (segment (start 77.7625 106.95) (end 76.897183 106.95) (width 0.4) (layer "F.Cu") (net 15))
 (segment (start 76.897183 106.95) (end 75.4 108.447183) (width 0.4) (layer "F.Cu") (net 15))
 (segment (start 72.9 104.9) (end 68.8 104.9) (width 0.4) (layer "F.Cu") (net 5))
 (segment (start 72.902817 106.3) (end 73.225 105.977817) (width 0.4) (layer "F.Cu") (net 5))
 (segment (start 68.8 104.9) (end 68.7625 104.8625) (width 0.4) (layer "F.Cu") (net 5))
 (segment (start 72.0375 106.3) (end 72.902817 106.3) (width 0.4) (layer "F.Cu") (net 5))
 (segment (start 73.225 105.977817) (end 73.225 105.225) (width 0.4) (layer "F.Cu") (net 5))
 (segment (start 73.225 105.225) (end 72.9 104.9) (width 0.4) (layer "F.Cu") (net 5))
 (segment (start 68.7625 104.8625) (end 68.7625 104.05) (width 0.4) (layer "F.Cu") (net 5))
 (segment (start 75.0625 104.05) (end 75.0625 105.440317) (width 0.4) (layer "F.Cu") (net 7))
 (segment (start 72.902817 107.6) (end 72.0375 107.6) (width 0.4) (layer "F.Cu") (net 7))
 (segment (start 75.0625 105.440317) (end 72.902817 107.6) (width 0.4) (layer "F.Cu") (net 7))
 (segment (start 72.0375 108.9) (end 70.979594 108.9) (width 0.4) (layer "F.Cu") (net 9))
 (segment (start 70.304594 108.225) (end 70.3 108.225) (width 0.4) (layer "F.Cu") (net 9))
 (segment (start 70.979594 108.9) (end 70.304594 108.225) (width 0.4) (layer "F.Cu") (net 9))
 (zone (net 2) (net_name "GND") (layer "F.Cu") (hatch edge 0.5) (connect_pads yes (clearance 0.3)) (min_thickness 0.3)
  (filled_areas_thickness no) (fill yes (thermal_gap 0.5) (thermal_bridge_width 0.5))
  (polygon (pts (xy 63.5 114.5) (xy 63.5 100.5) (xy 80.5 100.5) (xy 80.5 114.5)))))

